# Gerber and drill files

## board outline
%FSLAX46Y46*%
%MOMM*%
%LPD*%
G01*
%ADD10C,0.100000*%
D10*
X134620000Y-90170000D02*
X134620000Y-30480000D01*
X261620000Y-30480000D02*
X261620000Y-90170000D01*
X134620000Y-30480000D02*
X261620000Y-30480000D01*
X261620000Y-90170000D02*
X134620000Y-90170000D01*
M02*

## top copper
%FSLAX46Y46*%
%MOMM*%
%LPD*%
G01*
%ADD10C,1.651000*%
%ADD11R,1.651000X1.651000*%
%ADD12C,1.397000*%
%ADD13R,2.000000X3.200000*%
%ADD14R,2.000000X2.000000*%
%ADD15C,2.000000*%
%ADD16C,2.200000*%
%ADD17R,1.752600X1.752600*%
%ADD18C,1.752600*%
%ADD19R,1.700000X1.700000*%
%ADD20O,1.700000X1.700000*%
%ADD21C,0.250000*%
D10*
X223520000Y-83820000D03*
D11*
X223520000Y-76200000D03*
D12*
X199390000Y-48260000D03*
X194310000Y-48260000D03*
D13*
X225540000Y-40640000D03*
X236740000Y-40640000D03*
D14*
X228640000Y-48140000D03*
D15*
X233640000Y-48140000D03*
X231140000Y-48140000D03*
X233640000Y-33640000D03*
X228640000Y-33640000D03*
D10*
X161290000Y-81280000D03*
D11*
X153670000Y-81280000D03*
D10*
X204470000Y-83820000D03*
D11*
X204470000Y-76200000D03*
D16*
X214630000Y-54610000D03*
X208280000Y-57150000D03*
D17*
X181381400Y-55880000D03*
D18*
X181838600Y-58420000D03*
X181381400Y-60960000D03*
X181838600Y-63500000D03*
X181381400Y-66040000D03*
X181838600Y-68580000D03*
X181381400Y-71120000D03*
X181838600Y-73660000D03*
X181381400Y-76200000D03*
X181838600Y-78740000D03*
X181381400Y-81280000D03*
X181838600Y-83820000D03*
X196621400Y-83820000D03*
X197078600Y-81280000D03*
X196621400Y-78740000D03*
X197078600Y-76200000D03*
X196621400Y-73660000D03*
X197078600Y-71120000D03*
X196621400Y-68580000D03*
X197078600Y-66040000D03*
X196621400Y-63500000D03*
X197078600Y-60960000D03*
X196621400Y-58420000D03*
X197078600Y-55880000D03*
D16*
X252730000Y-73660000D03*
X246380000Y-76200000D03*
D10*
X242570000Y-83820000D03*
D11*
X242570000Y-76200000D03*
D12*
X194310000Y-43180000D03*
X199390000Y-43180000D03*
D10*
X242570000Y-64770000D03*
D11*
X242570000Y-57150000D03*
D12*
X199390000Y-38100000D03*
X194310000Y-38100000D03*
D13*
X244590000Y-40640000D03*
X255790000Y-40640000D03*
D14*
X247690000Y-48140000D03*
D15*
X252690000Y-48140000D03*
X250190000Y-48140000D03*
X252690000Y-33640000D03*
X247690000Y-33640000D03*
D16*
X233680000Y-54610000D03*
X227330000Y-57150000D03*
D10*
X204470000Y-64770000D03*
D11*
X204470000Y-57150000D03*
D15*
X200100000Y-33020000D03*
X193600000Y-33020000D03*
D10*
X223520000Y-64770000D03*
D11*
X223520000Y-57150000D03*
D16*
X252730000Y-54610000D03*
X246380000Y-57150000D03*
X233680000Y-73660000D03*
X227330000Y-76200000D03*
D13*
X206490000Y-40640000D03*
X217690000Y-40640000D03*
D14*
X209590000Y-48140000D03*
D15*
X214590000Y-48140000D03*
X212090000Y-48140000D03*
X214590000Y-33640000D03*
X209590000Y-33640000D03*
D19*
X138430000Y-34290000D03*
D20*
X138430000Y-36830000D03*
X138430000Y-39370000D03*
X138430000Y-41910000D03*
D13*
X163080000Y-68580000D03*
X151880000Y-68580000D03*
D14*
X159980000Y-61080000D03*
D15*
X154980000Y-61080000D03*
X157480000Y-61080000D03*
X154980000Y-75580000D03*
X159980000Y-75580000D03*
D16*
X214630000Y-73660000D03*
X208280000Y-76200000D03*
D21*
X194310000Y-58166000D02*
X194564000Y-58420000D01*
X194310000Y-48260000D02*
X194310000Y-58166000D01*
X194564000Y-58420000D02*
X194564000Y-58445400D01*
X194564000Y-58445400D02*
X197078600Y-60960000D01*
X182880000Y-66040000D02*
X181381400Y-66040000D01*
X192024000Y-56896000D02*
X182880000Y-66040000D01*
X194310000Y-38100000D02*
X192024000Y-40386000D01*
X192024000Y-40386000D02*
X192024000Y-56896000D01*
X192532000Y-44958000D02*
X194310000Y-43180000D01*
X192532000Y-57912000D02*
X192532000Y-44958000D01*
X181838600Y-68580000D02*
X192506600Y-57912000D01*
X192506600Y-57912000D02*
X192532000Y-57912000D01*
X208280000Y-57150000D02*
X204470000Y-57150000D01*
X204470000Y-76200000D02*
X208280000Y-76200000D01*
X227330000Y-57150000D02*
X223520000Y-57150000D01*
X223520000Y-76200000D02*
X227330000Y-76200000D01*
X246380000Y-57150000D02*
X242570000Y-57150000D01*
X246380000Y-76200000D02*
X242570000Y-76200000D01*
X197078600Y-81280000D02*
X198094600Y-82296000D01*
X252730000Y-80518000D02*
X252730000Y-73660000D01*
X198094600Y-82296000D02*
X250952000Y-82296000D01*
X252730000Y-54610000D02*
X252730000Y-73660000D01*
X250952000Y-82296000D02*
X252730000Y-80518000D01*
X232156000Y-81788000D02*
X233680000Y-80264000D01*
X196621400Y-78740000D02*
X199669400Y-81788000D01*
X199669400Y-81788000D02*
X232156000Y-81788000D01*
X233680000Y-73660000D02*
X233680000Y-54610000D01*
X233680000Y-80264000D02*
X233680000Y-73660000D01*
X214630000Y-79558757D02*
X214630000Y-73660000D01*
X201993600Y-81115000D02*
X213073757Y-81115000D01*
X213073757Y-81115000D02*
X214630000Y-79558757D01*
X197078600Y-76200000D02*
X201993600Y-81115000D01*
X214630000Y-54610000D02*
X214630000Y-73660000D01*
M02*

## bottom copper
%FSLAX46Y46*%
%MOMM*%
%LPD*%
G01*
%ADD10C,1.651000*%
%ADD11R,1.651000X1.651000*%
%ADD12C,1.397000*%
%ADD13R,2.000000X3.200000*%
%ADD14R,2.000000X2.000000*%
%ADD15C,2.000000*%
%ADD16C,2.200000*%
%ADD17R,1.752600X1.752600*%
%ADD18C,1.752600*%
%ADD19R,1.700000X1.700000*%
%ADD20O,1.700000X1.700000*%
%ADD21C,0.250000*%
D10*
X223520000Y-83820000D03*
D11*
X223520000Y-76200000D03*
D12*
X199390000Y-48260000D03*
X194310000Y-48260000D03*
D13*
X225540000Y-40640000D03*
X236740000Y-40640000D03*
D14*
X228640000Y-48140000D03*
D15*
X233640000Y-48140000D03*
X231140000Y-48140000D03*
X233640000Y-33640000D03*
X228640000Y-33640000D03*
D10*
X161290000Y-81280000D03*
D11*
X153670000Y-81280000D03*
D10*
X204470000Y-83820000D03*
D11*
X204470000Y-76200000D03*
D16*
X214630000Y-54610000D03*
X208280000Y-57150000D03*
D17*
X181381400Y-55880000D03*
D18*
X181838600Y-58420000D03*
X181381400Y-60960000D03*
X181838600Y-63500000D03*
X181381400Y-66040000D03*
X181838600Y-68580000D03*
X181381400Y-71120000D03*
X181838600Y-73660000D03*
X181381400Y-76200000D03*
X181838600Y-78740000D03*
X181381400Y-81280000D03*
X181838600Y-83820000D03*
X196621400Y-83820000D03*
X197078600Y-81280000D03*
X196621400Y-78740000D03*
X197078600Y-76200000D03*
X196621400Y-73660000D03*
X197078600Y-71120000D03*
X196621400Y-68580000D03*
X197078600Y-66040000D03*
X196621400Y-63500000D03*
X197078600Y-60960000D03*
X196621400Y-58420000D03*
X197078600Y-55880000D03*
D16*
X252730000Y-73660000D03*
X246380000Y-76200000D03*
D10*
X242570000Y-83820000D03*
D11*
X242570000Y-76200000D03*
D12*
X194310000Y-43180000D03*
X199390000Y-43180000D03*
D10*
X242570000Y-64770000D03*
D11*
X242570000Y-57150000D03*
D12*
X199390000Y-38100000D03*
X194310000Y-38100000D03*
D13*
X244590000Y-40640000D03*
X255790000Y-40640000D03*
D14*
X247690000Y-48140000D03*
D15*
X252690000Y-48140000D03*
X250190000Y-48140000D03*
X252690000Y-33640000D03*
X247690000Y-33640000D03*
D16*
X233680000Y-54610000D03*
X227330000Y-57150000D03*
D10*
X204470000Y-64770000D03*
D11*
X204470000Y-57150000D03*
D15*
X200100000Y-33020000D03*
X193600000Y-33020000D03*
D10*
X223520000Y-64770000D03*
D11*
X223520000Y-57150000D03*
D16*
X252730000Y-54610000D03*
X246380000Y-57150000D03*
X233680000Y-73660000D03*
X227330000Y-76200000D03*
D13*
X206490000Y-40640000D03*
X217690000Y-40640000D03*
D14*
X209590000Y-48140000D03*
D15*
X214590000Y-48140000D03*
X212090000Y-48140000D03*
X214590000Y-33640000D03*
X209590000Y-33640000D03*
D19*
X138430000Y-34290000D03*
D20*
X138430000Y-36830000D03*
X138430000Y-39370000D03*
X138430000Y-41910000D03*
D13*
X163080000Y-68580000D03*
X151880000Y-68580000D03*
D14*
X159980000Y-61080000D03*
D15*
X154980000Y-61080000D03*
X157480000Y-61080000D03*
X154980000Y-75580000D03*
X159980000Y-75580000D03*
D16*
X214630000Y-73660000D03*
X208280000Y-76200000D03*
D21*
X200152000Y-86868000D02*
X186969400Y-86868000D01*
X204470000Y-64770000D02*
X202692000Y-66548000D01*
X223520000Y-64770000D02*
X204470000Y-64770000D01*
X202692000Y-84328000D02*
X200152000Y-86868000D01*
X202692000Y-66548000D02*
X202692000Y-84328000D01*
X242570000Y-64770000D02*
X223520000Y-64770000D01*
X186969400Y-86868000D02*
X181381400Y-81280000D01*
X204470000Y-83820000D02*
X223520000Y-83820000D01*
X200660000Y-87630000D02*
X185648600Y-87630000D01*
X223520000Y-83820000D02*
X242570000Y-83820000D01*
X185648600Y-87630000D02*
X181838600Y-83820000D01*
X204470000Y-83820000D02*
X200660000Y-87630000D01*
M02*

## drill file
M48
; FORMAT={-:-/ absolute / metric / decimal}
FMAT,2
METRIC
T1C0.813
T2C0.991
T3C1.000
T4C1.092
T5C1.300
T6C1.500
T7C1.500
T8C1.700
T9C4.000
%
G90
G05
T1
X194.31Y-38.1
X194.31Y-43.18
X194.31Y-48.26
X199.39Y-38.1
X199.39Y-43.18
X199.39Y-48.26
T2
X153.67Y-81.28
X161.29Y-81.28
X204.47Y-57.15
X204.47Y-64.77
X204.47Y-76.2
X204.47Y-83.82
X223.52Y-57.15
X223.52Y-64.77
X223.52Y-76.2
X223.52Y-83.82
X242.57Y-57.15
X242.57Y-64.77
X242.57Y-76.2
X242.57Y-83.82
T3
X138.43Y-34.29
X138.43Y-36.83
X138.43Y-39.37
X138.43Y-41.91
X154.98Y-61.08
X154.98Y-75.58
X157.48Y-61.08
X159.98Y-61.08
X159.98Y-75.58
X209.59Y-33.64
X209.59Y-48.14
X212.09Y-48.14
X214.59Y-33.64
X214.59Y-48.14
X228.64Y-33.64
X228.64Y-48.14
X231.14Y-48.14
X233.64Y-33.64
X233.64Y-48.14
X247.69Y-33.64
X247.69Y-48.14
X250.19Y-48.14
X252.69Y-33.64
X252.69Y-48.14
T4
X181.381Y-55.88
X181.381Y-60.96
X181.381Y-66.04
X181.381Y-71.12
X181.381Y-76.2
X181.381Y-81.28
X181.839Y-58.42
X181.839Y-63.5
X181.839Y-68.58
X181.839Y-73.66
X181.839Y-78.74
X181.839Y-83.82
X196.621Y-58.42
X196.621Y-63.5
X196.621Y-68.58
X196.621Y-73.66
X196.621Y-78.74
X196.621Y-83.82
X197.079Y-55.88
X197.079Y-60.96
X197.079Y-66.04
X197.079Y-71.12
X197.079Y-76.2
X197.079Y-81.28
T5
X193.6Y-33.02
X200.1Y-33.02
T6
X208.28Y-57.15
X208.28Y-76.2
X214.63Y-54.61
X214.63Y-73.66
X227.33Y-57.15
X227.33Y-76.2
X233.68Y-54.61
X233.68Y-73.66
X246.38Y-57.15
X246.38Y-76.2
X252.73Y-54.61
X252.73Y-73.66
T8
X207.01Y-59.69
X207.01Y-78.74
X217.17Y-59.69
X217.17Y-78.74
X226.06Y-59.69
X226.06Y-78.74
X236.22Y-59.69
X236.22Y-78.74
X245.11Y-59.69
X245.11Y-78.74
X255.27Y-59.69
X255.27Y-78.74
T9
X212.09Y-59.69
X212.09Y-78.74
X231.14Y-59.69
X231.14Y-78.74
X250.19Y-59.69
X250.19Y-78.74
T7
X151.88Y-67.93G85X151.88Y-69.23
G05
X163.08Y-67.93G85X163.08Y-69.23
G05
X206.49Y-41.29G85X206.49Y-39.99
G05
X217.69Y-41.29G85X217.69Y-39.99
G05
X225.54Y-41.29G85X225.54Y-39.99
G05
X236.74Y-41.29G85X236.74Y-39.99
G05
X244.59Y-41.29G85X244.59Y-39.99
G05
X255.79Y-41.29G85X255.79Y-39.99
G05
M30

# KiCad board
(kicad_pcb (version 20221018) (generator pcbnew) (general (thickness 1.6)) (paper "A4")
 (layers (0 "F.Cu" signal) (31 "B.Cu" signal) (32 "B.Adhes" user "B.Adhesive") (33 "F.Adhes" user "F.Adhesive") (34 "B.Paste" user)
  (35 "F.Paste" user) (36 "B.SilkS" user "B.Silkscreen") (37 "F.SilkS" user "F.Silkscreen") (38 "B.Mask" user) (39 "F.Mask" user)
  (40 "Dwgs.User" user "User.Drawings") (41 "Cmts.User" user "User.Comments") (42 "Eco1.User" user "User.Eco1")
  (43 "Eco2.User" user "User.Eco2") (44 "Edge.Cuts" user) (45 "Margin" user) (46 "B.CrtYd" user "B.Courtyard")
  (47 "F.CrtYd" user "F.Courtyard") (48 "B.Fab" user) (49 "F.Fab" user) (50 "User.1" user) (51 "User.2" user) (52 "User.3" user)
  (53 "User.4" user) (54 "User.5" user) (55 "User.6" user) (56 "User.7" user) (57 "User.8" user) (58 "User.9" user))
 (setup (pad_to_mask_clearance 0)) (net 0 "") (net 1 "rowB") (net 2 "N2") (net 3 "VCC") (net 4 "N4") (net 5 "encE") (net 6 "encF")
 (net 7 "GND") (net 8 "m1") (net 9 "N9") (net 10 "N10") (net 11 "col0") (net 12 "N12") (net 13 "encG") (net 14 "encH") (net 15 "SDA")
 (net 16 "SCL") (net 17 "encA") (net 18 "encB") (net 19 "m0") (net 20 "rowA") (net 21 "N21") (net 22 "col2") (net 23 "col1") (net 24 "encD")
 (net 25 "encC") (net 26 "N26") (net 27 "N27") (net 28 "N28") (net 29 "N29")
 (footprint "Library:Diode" (layer "F.Cu") (at 223.52 80.01 90)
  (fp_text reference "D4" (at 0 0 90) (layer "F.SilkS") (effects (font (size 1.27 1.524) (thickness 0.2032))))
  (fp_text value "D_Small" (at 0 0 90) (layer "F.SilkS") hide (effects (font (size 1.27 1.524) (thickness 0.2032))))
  (pad "1" thru_hole circle (at -3.81 0 90) (size 1.651 1.651) (drill 0.9906) (layers "*.Cu" "*.SilkS" "*.Mask") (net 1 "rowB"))
  (pad "2" thru_hole rect (at 3.81 0 90) (size 1.651 1.651) (drill 0.9906) (layers "*.Cu" "*.SilkS" "*.Mask") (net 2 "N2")))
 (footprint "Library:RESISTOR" (layer "F.Cu") (at 196.85 48.26 180)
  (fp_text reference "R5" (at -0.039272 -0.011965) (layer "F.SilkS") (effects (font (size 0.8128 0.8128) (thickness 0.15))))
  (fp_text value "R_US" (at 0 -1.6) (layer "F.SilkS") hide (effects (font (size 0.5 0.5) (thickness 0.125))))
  (pad "1" thru_hole circle (at -2.54 0 180) (size 1.397 1.397) (drill 0.8128) (layers "*.Cu" "*.Mask") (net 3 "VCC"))
  (pad "2" thru_hole circle (at 2.54 0 180) (size 1.397 1.397) (drill 0.8128) (layers "*.Cu" "*.Mask") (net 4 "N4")))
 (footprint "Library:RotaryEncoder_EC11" (layer "F.Cu") (at 231.14 40.64 90)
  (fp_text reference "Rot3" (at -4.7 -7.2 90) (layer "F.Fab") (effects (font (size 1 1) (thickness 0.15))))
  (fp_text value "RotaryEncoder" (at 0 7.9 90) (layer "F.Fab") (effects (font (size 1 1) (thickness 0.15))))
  (pad "" np_thru_hole rect (at 0 -5.6 90) (size 3.2 2) (drill oval 2.8 1.5) (layers "*.Cu" "*.Mask"))
  (pad "" np_thru_hole rect (at 0 5.6 90) (size 3.2 2) (drill oval 2.8 1.5) (layers "*.Cu" "*.Mask"))
  (pad "A" thru_hole rect (at -7.5 -2.5 90) (size 2 2) (drill 1) (layers "*.Cu" "*.Mask") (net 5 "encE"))
  (pad "B" thru_hole circle (at -7.5 2.5 90) (size 2 2) (drill 1) (layers "*.Cu" "*.Mask") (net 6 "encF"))
  (pad "C" thru_hole circle (at -7.5 0 90) (size 2 2) (drill 1) (layers "*.Cu" "*.Mask") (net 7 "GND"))
  (pad "S1" thru_hole circle (at 7 2.5 90) (size 2 2) (drill 1) (layers "*.Cu" "*.Mask"))
  (pad "S2" thru_hole circle (at 7 -2.5 90) (size 2 2) (drill 1) (layers "*.Cu" "*.Mask")))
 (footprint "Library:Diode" (layer "F.Cu") (at 157.48 81.28 180)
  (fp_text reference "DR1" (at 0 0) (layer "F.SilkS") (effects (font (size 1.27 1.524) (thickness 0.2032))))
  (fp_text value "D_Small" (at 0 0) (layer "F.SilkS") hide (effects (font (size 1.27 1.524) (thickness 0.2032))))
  (pad "1" thru_hole circle (at -3.81 0 180) (size 1.651 1.651) (drill 0.9906) (layers "*.Cu" "*.SilkS" "*.Mask") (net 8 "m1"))
  (pad "2" thru_hole rect (at 3.81 0 180) (size 1.651 1.651) (drill 0.9906) (layers "*.Cu" "*.SilkS" "*.Mask") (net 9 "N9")))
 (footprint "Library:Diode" (layer "F.Cu") (at 204.47 80.01 90)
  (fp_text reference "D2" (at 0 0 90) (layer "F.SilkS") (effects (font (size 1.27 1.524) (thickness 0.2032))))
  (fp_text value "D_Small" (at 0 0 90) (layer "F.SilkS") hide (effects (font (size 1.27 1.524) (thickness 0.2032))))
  (pad "1" thru_hole circle (at -3.81 0 90) (size 1.651 1.651) (drill 0.9906) (layers "*.Cu" "*.SilkS" "*.Mask") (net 1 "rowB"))
  (pad "2" thru_hole rect (at 3.81 0 90) (size 1.651 1.651) (drill 0.9906) (layers "*.Cu" "*.SilkS" "*.Mask") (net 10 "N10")))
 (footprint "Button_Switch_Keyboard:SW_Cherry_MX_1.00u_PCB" (layer "F.Cu") (at 214.63 54.61)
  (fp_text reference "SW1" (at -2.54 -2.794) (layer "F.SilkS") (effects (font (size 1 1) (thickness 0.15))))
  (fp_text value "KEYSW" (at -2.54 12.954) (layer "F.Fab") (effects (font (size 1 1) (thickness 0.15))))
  (pad "" np_thru_hole circle (at -7.62 5.08) (size 1.7 1.7) (drill 1.7) (layers "*.Cu" "*.Mask"))
  (pad "" np_thru_hole circle (at -2.54 5.08) (size 4 4) (drill 4) (layers "*.Cu" "*.Mask"))
  (pad "" np_thru_hole circle (at 2.54 5.08) (size 1.7 1.7) (drill 1.7) (layers "*.Cu" "*.Mask"))
  (pad "1" thru_hole circle (at 0 0) (size 2.2 2.2) (drill 1.5) (layers "*.Cu" "*.Mask") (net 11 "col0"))
  (pad "2" thru_hole circle (at -6.35 2.54) (size 2.2 2.2) (drill 1.5) (layers "*.Cu" "*.Mask") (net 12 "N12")))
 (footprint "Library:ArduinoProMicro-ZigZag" (layer "F.Cu") (at 189.23 69.85 -90)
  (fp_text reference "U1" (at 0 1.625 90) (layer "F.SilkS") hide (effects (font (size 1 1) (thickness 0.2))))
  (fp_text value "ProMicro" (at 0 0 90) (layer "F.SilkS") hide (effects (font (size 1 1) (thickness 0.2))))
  (pad "1" thru_hole rect (at -13.97 7.8486 270) (size 1.7526 1.7526) (drill 1.0922) (layers "*.Cu" "*.SilkS" "*.Mask") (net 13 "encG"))
  (pad "2" thru_hole circle (at -11.43 7.3914 270) (size 1.7526 1.7526) (drill 1.0922) (layers "*.Cu" "*.SilkS" "*.Mask") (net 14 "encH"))
  (pad "3" thru_hole circle (at -8.89 7.8486 270) (size 1.7526 1.7526) (drill 1.0922) (layers "*.Cu" "*.SilkS" "*.Mask") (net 7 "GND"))
  (pad "4" thru_hole circle (at -6.35 7.3914 270) (size 1.7526 1.7526) (drill 1.0922) (layers "*.Cu" "*.SilkS" "*.Mask") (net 7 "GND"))
  (pad "5" thru_hole circle (at -3.81 7.8486 270) (size 1.7526 1.7526) (drill 1.0922) (layers "*.Cu" "*.SilkS" "*.Mask") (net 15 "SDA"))
  (pad "6" thru_hole circle (at -1.27 7.3914 270) (size 1.7526 1.7526) (drill 1.0922) (layers "*.Cu" "*.SilkS" "*.Mask") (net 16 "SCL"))
  (pad "7" thru_hole circle (at 1.27 7.8486 270) (size 1.7526 1.7526) (drill 1.0922) (layers "*.Cu" "*.SilkS" "*.Mask") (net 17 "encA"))
  (pad "8" thru_hole circle (at 3.81 7.3914 270) (size 1.7526 1.7526) (drill 1.0922) (layers "*.Cu" "*.SilkS" "*.Mask") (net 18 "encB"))
  (pad "9" thru_hole circle (at 6.35 7.8486 270) (size 1.7526 1.7526) (drill 1.0922) (layers "*.Cu" "*.SilkS" "*.Mask") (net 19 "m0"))
  (pad "10" thru_hole circle (at 8.89 7.3914 270) (size 1.7526 1.7526) (drill 1.0922) (layers "*.Cu" "*.SilkS" "*.Mask") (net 8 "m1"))
  (pad "11" thru_hole circle (at 11.43 7.8486 270) (size 1.7526 1.7526) (drill 1.0922) (layers "*.Cu" "*.SilkS" "*.Mask") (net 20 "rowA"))
  (pad "12" thru_hole circle (at 13.97 7.3914 270) (size 1.7526 1.7526) (drill 1.0922) (layers "*.Cu" "*.SilkS" "*.Mask") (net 1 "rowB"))
  (pad "13" thru_hole circle (at 13.97 -7.3914 270) (size 1.7526 1.7526) (drill 1.0922) (layers "*.Cu" "*.SilkS" "*.Mask") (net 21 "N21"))
  (pad "14" thru_hole circle (at 11.43 -7.8486 270) (size 1.7526 1.7526) (drill 1.0922) (layers "*.Cu" "*.SilkS" "*.Mask") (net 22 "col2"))
  (pad "15" thru_hole circle (at 8.89 -7.3914 270) (size 1.7526 1.7526) (drill 1.0922) (layers "*.Cu" "*.SilkS" "*.Mask") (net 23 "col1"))
  (pad "16" thru_hole circle (at 6.35 -7.8486 270) (size 1.7526 1.7526) (drill 1.0922) (layers "*.Cu" "*.SilkS" "*.Mask") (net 11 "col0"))
  (pad "17" thru_hole circle (at 3.81 -7.3914 270) (size 1.7526 1.7526) (drill 1.0922) (layers "*.Cu" "*.SilkS" "*.Mask") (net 6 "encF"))
  (pad "18" thru_hole circle (at 1.27 -7.8486 270) (size 1.7526 1.7526) (drill 1.0922) (layers "*.Cu" "*.SilkS" "*.Mask") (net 5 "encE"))
  (pad "19" thru_hole circle (at -1.27 -7.3914 270) (size 1.7526 1.7526) (drill 1.0922) (layers "*.Cu" "*.SilkS" "*.Mask") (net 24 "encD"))
  (pad "20" thru_hole circle (at -3.81 -7.8486 270) (size 1.7526 1.7526) (drill 1.0922) (layers "*.Cu" "*.SilkS" "*.Mask") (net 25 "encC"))
  (pad "21" thru_hole circle (at -6.35 -7.3914 270) (size 1.7526 1.7526) (drill 1.0922) (layers "*.Cu" "*.SilkS" "*.Mask") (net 3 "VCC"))
  (pad "22" thru_hole circle (at -8.89 -7.8486 270) (size 1.7526 1.7526) (drill 1.0922) (layers "*.Cu" "*.SilkS" "*.Mask") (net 4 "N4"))
  (pad "23" thru_hole circle (at -11.43 -7.3914 270) (size 1.7526 1.7526) (drill 1.0922) (layers "*.Cu" "*.SilkS" "*.Mask") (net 7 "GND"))
  (pad "24" thru_hole circle (at -13.97 -7.8486 270) (size 1.7526 1.7526) (drill 1.0922) (layers "*.Cu" "*.SilkS" "*.Mask") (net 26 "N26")))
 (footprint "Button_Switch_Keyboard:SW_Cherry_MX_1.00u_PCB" (layer "F.Cu") (at 252.73 73.66)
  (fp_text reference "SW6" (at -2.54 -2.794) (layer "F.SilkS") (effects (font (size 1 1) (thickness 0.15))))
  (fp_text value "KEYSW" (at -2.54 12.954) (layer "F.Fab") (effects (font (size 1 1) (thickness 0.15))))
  (pad "" np_thru_hole circle (at -7.62 5.08) (size 1.7 1.7) (drill 1.7) (layers "*.Cu" "*.Mask"))
  (pad "" np_thru_hole circle (at -2.54 5.08) (size 4 4) (drill 4) (layers "*.Cu" "*.Mask"))
  (pad "" np_thru_hole circle (at 2.54 5.08) (size 1.7 1.7) (drill 1.7) (layers "*.Cu" "*.Mask"))
  (pad "1" thru_hole circle (at 0 0) (size 2.2 2.2) (drill 1.5) (layers "*.Cu" "*.Mask") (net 22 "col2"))
  (pad "2" thru_hole circle (at -6.35 2.54) (size 2.2 2.2) (drill 1.5) (layers "*.Cu" "*.Mask") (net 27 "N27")))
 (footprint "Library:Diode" (layer "F.Cu") (at 242.57 80.01 90)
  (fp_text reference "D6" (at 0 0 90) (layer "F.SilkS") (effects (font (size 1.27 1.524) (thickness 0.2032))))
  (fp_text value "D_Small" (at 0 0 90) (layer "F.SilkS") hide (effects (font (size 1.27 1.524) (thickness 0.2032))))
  (pad "1" thru_hole circle (at -3.81 0 90) (size 1.651 1.651) (drill 0.9906) (layers "*.Cu" "*.SilkS" "*.Mask") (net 1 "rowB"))
  (pad "2" thru_hole rect (at 3.81 0 90) (size 1.651 1.651) (drill 0.9906) (layers "*.Cu" "*.SilkS" "*.Mask") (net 27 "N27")))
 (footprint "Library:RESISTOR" (layer "F.Cu") (at 196.85 43.18)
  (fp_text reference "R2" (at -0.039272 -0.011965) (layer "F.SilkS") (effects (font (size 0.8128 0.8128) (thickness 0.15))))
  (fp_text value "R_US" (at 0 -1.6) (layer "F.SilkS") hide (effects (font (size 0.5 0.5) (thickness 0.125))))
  (pad "1" thru_hole circle (at -2.54 0) (size 1.397 1.397) (drill 0.8128) (layers "*.Cu" "*.Mask") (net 16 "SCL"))
  (pad "2" thru_hole circle (at 2.54 0) (size 1.397 1.397) (drill 0.8128) (layers "*.Cu" "*.Mask") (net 3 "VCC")))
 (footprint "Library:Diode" (layer "F.Cu") (at 242.57 60.96 90)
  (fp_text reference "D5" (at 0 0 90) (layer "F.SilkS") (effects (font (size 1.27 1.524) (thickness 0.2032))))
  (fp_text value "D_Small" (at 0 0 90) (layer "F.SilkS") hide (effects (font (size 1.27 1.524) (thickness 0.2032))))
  (pad "1" thru_hole circle (at -3.81 0 90) (size 1.651 1.651) (drill 0.9906) (layers "*.Cu" "*.SilkS" "*.Mask") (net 20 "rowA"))
  (pad "2" thru_hole rect (at 3.81 0 90) (size 1.651 1.651) (drill 0.9906) (layers "*.Cu" "*.SilkS" "*.Mask") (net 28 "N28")))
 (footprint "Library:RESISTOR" (layer "F.Cu") (at 196.85 38.1 180)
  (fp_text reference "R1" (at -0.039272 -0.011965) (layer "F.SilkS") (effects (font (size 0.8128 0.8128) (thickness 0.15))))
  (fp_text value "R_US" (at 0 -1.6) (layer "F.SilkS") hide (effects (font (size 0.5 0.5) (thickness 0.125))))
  (pad "1" thru_hole circle (at -2.54 0 180) (size 1.397 1.397) (drill 0.8128) (layers "*.Cu" "*.Mask") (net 3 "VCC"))
  (pad "2" thru_hole circle (at 2.54 0 180) (size 1.397 1.397) (drill 0.8128) (layers "*.Cu" "*.Mask") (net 15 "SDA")))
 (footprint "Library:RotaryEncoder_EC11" (layer "F.Cu") (at 250.19 40.64 90)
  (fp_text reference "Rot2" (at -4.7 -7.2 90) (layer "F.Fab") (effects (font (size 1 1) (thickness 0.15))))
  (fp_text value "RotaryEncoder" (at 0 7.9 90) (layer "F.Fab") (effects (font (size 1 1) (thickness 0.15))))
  (pad "" np_thru_hole rect (at 0 -5.6 90) (size 3.2 2) (drill oval 2.8 1.5) (layers "*.Cu" "*.Mask"))
  (pad "" np_thru_hole rect (at 0 5.6 90) (size 3.2 2) (drill oval 2.8 1.5) (layers "*.Cu" "*.Mask"))
  (pad "A" thru_hole rect (at -7.5 -2.5 90) (size 2 2) (drill 1) (layers "*.Cu" "*.Mask") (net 25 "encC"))
  (pad "B" thru_hole circle (at -7.5 2.5 90) (size 2 2) (drill 1) (layers "*.Cu" "*.Mask") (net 24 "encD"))
  (pad "C" thru_hole circle (at -7.5 0 90) (size 2 2) (drill 1) (layers "*.Cu" "*.Mask") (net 7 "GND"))
  (pad "S1" thru_hole circle (at 7 2.5 90) (size 2 2) (drill 1) (layers "*.Cu" "*.Mask"))
  (pad "S2" thru_hole circle (at 7 -2.5 90) (size 2 2) (drill 1) (layers "*.Cu" "*.Mask")))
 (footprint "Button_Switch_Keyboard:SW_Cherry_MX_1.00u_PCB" (layer "F.Cu") (at 233.68 54.61)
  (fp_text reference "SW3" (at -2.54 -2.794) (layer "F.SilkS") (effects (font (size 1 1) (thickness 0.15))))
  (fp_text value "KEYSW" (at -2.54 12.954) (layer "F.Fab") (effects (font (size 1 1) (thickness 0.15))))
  (pad "" np_thru_hole circle (at -7.62 5.08) (size 1.7 1.7) (drill 1.7) (layers "*.Cu" "*.Mask"))
  (pad "" np_thru_hole circle (at -2.54 5.08) (size 4 4) (drill 4) (layers "*.Cu" "*.Mask"))
  (pad "" np_thru_hole circle (at 2.54 5.08) (size 1.7 1.7) (drill 1.7) (layers "*.Cu" "*.Mask"))
  (pad "1" thru_hole circle (at 0 0) (size 2.2 2.2) (drill 1.5) (layers "*.Cu" "*.Mask") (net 23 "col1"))
  (pad "2" thru_hole circle (at -6.35 2.54) (size 2.2 2.2) (drill 1.5) (layers "*.Cu" "*.Mask") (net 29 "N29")))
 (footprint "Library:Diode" (layer "F.Cu") (at 204.47 60.96 90)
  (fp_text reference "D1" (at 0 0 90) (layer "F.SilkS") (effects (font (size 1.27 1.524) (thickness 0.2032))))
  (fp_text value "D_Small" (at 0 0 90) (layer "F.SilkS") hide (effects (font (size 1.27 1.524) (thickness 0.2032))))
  (pad "1" thru_hole circle (at -3.81 0 90) (size 1.651 1.651) (drill 0.9906) (layers "*.Cu" "*.SilkS" "*.Mask") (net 20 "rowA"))
  (pad "2" thru_hole rect (at 3.81 0 90) (size 1.651 1.651) (drill 0.9906) (layers "*.Cu" "*.SilkS" "*.Mask") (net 12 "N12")))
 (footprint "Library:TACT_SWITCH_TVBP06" (layer "F.Cu") (at 196.85 33.02 180)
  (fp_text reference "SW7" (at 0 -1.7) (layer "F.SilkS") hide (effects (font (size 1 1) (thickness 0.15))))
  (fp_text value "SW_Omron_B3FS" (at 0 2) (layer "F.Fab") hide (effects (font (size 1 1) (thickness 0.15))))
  (pad "1" thru_hole circle (at -3.25 0 180) (size 2 2) (drill 1.3) (layers "*.Cu" "*.Mask") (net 7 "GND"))
  (pad "2" thru_hole circle (at 3.25 0 180) (size 2 2) (drill 1.3) (layers "*.Cu" "*.Mask") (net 4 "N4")))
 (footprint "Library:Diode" (layer "F.Cu") (at 223.52 60.96 90)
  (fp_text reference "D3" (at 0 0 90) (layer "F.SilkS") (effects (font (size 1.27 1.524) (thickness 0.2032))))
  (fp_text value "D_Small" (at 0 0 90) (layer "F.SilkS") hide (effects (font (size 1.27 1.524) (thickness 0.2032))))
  (pad "1" thru_hole circle (at -3.81 0 90) (size 1.651 1.651) (drill 0.9906) (layers "*.Cu" "*.SilkS" "*.Mask") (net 20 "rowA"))
  (pad "2" thru_hole rect (at 3.81 0 90) (size 1.651 1.651) (drill 0.9906) (layers "*.Cu" "*.SilkS" "*.Mask") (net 29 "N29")))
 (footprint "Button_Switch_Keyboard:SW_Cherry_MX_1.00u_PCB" (layer "F.Cu") (at 252.73 54.61)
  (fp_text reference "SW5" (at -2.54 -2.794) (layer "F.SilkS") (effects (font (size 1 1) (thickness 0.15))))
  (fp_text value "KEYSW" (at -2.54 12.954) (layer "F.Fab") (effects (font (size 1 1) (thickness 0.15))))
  (pad "" np_thru_hole circle (at -7.62 5.08) (size 1.7 1.7) (drill 1.7) (layers "*.Cu" "*.Mask"))
  (pad "" np_thru_hole circle (at -2.54 5.08) (size 4 4) (drill 4) (layers "*.Cu" "*.Mask"))
  (pad "" np_thru_hole circle (at 2.54 5.08) (size 1.7 1.7) (drill 1.7) (layers "*.Cu" "*.Mask"))
  (pad "1" thru_hole circle (at 0 0) (size 2.2 2.2) (drill 1.5) (layers "*.Cu" "*.Mask") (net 22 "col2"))
  (pad "2" thru_hole circle (at -6.35 2.54) (size 2.2 2.2) (drill 1.5) (layers "*.Cu" "*.Mask") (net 28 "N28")))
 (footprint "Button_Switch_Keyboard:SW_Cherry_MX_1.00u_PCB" (layer "F.Cu") (at 233.68 73.66)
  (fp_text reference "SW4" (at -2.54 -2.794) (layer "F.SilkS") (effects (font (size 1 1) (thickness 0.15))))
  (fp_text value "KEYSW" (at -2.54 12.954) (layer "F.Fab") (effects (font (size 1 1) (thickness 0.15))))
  (pad "" np_thru_hole circle (at -7.62 5.08) (size 1.7 1.7) (drill 1.7) (layers "*.Cu" "*.Mask"))
  (pad "" np_thru_hole circle (at -2.54 5.08) (size 4 4) (drill 4) (layers "*.Cu" "*.Mask"))
  (pad "" np_thru_hole circle (at 2.54 5.08) (size 1.7 1.7) (drill 1.7) (layers "*.Cu" "*.Mask"))
  (pad "1" thru_hole circle (at 0 0) (size 2.2 2.2) (drill 1.5) (layers "*.Cu" "*.Mask") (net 23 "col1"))
  (pad "2" thru_hole circle (at -6.35 2.54) (size 2.2 2.2) (drill 1.5) (layers "*.Cu" "*.Mask") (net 2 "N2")))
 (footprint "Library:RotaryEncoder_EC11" (layer "F.Cu") (at 212.09 40.64 90)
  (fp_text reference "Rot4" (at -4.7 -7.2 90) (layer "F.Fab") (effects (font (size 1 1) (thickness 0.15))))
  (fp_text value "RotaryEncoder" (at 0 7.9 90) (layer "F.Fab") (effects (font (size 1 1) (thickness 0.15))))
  (pad "" np_thru_hole rect (at 0 -5.6 90) (size 3.2 2) (drill oval 2.8 1.5) (layers "*.Cu" "*.Mask"))
  (pad "" np_thru_hole rect (at 0 5.6 90) (size 3.2 2) (drill oval 2.8 1.5) (layers "*.Cu" "*.Mask"))
  (pad "A" thru_hole rect (at -7.5 -2.5 90) (size 2 2) (drill 1) (layers "*.Cu" "*.Mask") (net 13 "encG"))
  (pad "B" thru_hole circle (at -7.5 2.5 90) (size 2 2) (drill 1) (layers "*.Cu" "*.Mask") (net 14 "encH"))
  (pad "C" thru_hole circle (at -7.5 0 90) (size 2 2) (drill 1) (layers "*.Cu" "*.Mask") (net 7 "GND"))
  (pad "S1" thru_hole circle (at 7 2.5 90) (size 2 2) (drill 1) (layers "*.Cu" "*.Mask"))
  (pad "S2" thru_hole circle (at 7 -2.5 90) (size 2 2) (drill 1) (layers "*.Cu" "*.Mask")))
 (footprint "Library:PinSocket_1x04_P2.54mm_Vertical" (layer "F.Cu") (at 138.43 34.29)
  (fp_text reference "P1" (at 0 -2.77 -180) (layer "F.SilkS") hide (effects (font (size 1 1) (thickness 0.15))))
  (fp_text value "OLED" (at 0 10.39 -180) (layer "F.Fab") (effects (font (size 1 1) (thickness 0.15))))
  (pad "1" thru_hole rect (at 0 0) (size 1.7 1.7) (drill 1) (layers "*.Cu" "*.Mask") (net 7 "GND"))
  (pad "2" thru_hole oval (at 0 2.54) (size 1.7 1.7) (drill 1) (layers "*.Cu" "*.Mask") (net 3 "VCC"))
  (pad "3" thru_hole oval (at 0 5.08) (size 1.7 1.7) (drill 1) (layers "*.Cu" "*.Mask") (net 16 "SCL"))
  (pad "4" thru_hole oval (at 0 7.62) (size 1.7 1.7) (drill 1) (layers "*.Cu" "*.Mask") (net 15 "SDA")))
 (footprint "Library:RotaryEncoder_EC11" (layer "F.Cu") (at 157.48 68.58 -90)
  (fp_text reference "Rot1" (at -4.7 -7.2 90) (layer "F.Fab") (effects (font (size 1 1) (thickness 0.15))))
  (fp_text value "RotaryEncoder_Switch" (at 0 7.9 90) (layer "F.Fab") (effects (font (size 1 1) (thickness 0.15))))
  (pad "" np_thru_hole rect (at 0 -5.6 270) (size 3.2 2) (drill oval 2.8 1.5) (layers "*.Cu" "*.Mask"))
  (pad "" np_thru_hole rect (at 0 5.6 270) (size 3.2 2) (drill oval 2.8 1.5) (layers "*.Cu" "*.Mask"))
  (pad "A" thru_hole rect (at -7.5 -2.5 270) (size 2 2) (drill 1) (layers "*.Cu" "*.Mask") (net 17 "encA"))
  (pad "B" thru_hole circle (at -7.5 2.5 270) (size 2 2) (drill 1) (layers "*.Cu" "*.Mask") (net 18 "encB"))
  (pad "C" thru_hole circle (at -7.5 0 270) (size 2 2) (drill 1) (layers "*.Cu" "*.Mask") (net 7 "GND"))
  (pad "S1" thru_hole circle (at 7 2.5 270) (size 2 2) (drill 1) (layers "*.Cu" "*.Mask") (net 19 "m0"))
  (pad "S2" thru_hole circle (at 7 -2.5 270) (size 2 2) (drill 1) (layers "*.Cu" "*.Mask") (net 9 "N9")))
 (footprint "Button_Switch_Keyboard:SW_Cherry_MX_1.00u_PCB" (layer "F.Cu") (at 214.63 73.66)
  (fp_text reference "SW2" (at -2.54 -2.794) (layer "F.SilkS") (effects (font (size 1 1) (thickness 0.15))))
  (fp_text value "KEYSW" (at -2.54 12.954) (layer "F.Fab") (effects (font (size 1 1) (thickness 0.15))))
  (pad "" np_thru_hole circle (at -7.62 5.08) (size 1.7 1.7) (drill 1.7) (layers "*.Cu" "*.Mask"))
  (pad "" np_thru_hole circle (at -2.54 5.08) (size 4 4) (drill 4) (layers "*.Cu" "*.Mask"))
  (pad "" np_thru_hole circle (at 2.54 5.08) (size 1.7 1.7) (drill 1.7) (layers "*.Cu" "*.Mask"))
  (pad "1" thru_hole circle (at 0 0) (size 2.2 2.2) (drill 1.5) (layers "*.Cu" "*.Mask") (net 11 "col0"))
  (pad "2" thru_hole circle (at -6.35 2.54) (size 2.2 2.2) (drill 1.5) (layers "*.Cu" "*.Mask") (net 10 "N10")))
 (gr_line (start 134.62 90.17) (end 134.62 30.48) (stroke (width 0.1) (type default)) (layer "Edge.Cuts"))
 (gr_line (start 261.62 30.48) (end 261.62 90.17) (stroke (width 0.1) (type default)) (layer "Edge.Cuts"))
 (gr_line (start 134.62 30.48) (end 261.62 30.48) (stroke (width 0.1) (type default)) (layer "Edge.Cuts"))
 (gr_line (start 261.62 90.17) (end 134.62 90.17) (stroke (width 0.1) (type default)) (layer "Edge.Cuts"))
 (segment (start 194.31 58.166) (end 194.564 58.42) (width 0.25) (layer "F.Cu") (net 4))
 (segment (start 194.31 48.26) (end 194.31 58.166) (width 0.25) (layer "F.Cu") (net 4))
 (segment (start 194.564 58.42) (end 194.564 58.4454) (width 0.25) (layer "F.Cu") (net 4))
 (segment (start 194.564 58.4454) (end 197.0786 60.96) (width 0.25) (layer "F.Cu") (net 4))
 (segment (start 182.88 66.04) (end 181.3814 66.04) (width 0.25) (layer "F.Cu") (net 15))
 (segment (start 192.024 56.896) (end 182.88 66.04) (width 0.25) (layer "F.Cu") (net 15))
 (segment (start 194.31 38.1) (end 192.024 40.386) (width 0.25) (layer "F.Cu") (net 15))
 (segment (start 192.024 40.386) (end 192.024 56.896) (width 0.25) (layer "F.Cu") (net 15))
 (segment (start 192.532 44.958) (end 194.31 43.18) (width 0.25) (layer "F.Cu") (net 16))
 (segment (start 192.532 57.912) (end 192.532 44.958) (width 0.25) (layer "F.Cu") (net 16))
 (segment (start 181.8386 68.58) (end 192.5066 57.912) (width 0.25) (layer "F.Cu") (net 16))
 (segment (start 192.5066 57.912) (end 192.532 57.912) (width 0.25) (layer "F.Cu") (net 16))
 (segment (start 200.152 86.868) (end 186.9694 86.868) (width 0.25) (layer "B.Cu") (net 20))
 (segment (start 204.47 64.77) (end 202.692 66.548) (width 0.25) (layer "B.Cu") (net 20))
 (segment (start 223.52 64.77) (end 204.47 64.77) (width 0.25) (layer "B.Cu") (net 20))
 (segment (start 202.692 84.328) (end 200.152 86.868) (width 0.25) (layer "B.Cu") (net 20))
 (segment (start 202.692 66.548) (end 202.692 84.328) (width 0.25) (layer "B.Cu") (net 20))
 (segment (start 242.57 64.77) (end 223.52 64.77) (width 0.25) (layer "B.Cu") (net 20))
 (segment (start 186.9694 86.868) (end 181.3814 81.28) (width 0.25) (layer "B.Cu") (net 20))
 (segment (start 208.28 57.15) (end 204.47 57.15) (width 0.25) (layer "F.Cu") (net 12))
 (segment (start 204.47 83.82) (end 223.52 83.82) (width 0.25) (layer "B.Cu") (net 1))
 (segment (start 200.66 87.63) (end 185.6486 87.63) (width 0.25) (layer "B.Cu") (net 1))
 (segment (start 223.52 83.82) (end 242.57 83.82) (width 0.25) (layer "B.Cu") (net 1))
 (segment (start 185.6486 87.63) (end 181.8386 83.82) (width 0.25) (layer "B.Cu") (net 1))
 (segment (start 204.47 83.82) (end 200.66 87.63) (width 0.25) (layer "B.Cu") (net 1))
 (segment (start 204.47 76.2) (end 208.28 76.2) (width 0.25) (layer "F.Cu") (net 10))
 (segment (start 227.33 57.15) (end 223.52 57.15) (width 0.25) (layer "F.Cu") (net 29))
 (segment (start 223.52 76.2) (end 227.33 76.2) (width 0.25) (layer "F.Cu") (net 2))
 (segment (start 246.38 57.15) (end 242.57 57.15) (width 0.25) (layer "F.Cu") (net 28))
 (segment (start 246.38 76.2) (end 242.57 76.2) (width 0.25) (layer "F.Cu") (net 27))
 (segment (start 197.0786 81.28) (end 198.0946 82.296) (width 0.25) (layer "F.Cu") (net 22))
 (segment (start 252.73 80.518) (end 252.73 73.66) (width 0.25) (layer "F.Cu") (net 22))
 (segment (start 198.0946 82.296) (end 250.952 82.296) (width 0.25) (layer "F.Cu") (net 22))
 (segment (start 252.73 54.61) (end 252.73 73.66) (width 0.25) (layer "F.Cu") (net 22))
 (segment (start 250.952 82.296) (end 252.73 80.518) (width 0.25) (layer "F.Cu") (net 22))
 (segment (start 232.156 81.788) (end 233.68 80.264) (width 0.25) (layer "F.Cu") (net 23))
 (segment (start 196.6214 78.74) (end 199.6694 81.788) (width 0.25) (layer "F.Cu") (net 23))
 (segment (start 199.6694 81.788) (end 232.156 81.788) (width 0.25) (layer "F.Cu") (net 23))
 (segment (start 233.68 73.66) (end 233.68 54.61) (width 0.25) (layer "F.Cu") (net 23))
 (segment (start 233.68 80.264) (end 233.68 73.66) (width 0.25) (layer "F.Cu") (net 23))
 (segment (start 214.63 79.558757) (end 214.63 73.66) (width 0.25) (layer "F.Cu") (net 11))
 (segment (start 201.9936 81.115) (end 213.073757 81.115) (width 0.25) (layer "F.Cu") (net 11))
 (segment (start 213.073757 81.115) (end 214.63 79.558757) (width 0.25) (layer "F.Cu") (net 11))
 (segment (start 197.0786 76.2) (end 201.9936 81.115) (width 0.25) (layer "F.Cu") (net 11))
 (segment (start 214.63 54.61) (end 214.63 73.66) (width 0.25) (layer "F.Cu") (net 11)))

